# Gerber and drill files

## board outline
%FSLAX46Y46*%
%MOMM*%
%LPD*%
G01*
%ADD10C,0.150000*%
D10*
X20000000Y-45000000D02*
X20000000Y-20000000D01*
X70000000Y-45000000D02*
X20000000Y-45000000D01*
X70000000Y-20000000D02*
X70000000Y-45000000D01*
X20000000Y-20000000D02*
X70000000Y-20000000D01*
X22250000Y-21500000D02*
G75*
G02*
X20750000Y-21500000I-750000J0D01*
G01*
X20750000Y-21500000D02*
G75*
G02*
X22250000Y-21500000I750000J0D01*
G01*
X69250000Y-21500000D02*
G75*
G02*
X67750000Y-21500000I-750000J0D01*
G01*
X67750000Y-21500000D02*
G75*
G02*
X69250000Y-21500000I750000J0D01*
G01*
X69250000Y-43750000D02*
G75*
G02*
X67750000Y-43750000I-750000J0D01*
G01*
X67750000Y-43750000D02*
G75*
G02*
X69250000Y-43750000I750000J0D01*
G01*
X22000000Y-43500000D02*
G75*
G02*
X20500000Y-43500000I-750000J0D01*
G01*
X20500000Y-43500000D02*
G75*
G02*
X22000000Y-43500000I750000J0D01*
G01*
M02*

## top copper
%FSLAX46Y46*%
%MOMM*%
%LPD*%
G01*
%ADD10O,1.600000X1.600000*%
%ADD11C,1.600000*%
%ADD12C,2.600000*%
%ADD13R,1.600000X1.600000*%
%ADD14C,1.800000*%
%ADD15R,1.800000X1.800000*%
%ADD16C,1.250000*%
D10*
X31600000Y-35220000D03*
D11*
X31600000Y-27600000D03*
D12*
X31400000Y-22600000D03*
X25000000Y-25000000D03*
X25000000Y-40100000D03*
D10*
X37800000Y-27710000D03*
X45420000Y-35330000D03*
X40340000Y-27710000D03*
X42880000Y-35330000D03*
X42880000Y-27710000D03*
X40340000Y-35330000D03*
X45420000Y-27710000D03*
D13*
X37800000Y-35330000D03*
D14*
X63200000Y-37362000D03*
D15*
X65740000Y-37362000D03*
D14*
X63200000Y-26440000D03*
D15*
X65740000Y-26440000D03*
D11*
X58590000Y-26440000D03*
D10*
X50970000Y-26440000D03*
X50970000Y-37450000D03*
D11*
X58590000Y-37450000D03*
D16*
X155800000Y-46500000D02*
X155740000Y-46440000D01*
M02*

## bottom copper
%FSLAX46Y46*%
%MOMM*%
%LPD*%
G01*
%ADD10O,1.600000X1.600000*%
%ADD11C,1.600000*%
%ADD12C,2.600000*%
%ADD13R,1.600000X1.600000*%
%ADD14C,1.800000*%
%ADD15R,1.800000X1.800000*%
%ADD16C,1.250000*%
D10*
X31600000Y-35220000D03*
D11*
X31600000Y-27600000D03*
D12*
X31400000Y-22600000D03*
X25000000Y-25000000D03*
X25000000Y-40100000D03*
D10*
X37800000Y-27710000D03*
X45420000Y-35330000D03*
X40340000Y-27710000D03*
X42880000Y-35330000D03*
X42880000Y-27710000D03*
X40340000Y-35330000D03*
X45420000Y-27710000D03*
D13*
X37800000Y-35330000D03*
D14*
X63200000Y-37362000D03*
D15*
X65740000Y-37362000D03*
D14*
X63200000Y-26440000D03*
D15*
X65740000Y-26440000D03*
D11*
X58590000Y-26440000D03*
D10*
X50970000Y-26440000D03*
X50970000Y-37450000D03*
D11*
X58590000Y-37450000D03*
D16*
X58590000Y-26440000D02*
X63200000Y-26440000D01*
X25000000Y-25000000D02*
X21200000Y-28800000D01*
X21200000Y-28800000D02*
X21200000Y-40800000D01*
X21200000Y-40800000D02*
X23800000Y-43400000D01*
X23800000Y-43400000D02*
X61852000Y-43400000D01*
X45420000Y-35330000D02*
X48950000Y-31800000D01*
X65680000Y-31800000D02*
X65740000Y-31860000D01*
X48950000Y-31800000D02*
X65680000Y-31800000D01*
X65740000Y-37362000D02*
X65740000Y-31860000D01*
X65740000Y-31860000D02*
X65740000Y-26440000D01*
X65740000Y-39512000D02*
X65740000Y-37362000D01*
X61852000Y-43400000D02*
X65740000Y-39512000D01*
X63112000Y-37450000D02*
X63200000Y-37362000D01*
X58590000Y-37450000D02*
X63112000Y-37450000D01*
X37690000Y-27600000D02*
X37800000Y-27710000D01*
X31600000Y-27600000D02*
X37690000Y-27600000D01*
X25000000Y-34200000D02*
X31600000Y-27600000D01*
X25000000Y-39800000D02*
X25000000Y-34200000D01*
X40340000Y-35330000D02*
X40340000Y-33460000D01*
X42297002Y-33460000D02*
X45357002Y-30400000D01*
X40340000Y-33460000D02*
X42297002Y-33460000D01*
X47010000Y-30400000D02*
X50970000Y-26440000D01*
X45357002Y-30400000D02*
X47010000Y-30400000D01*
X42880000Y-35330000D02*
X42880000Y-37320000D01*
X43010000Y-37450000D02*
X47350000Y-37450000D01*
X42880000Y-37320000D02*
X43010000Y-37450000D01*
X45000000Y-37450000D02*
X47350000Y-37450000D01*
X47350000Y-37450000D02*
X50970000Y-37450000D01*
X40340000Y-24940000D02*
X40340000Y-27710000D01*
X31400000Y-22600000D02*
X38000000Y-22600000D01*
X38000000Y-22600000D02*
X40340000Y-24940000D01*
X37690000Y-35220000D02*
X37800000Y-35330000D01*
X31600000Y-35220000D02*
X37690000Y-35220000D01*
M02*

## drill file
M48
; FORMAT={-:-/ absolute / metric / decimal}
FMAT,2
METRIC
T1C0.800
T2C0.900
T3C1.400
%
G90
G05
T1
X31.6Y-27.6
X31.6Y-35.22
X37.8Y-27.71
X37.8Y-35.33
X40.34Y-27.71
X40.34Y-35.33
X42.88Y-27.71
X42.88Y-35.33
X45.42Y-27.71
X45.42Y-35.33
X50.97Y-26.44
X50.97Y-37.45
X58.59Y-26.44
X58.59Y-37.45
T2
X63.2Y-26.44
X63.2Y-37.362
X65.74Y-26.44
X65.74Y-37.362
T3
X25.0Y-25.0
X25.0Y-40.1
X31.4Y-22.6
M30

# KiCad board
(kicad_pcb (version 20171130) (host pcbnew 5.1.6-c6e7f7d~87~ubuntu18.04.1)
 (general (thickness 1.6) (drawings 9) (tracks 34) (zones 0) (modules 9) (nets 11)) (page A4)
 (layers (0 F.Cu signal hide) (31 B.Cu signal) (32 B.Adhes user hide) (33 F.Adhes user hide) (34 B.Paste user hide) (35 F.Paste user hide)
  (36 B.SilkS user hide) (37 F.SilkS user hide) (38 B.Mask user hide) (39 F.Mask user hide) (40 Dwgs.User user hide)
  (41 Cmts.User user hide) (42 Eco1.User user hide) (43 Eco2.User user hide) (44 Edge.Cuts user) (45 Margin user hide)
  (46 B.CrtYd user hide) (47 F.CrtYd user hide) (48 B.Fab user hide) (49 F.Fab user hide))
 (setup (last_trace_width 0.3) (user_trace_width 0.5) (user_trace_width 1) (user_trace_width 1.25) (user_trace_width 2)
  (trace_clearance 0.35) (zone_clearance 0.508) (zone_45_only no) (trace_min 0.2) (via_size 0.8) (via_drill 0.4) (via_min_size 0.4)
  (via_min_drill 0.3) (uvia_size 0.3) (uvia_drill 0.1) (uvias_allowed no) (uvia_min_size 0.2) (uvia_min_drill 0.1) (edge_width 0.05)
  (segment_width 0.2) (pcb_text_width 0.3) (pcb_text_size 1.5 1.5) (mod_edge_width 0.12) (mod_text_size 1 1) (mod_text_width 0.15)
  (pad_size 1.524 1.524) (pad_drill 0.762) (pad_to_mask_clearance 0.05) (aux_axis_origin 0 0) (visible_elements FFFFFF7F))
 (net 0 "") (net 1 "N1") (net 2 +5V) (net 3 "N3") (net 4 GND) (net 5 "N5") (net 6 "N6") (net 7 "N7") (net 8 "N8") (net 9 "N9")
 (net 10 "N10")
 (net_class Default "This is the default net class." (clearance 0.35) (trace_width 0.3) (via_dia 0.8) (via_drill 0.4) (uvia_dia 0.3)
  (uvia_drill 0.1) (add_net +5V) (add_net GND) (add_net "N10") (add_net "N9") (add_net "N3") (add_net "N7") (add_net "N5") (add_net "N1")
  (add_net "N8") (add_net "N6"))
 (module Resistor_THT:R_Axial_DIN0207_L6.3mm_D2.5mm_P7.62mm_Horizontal (layer F.Cu) (at 31.6 27.6 270)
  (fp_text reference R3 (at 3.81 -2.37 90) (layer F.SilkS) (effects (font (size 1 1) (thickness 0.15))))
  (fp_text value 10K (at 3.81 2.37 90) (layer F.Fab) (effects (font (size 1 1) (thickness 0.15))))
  (pad 2 thru_hole oval (at 7.62 0 270) (size 1.6 1.6) (drill 0.8) (layers *.Cu *.Mask) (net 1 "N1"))
  (pad 1 thru_hole circle (at 0 0 270) (size 1.6 1.6) (drill 0.8) (layers *.Cu *.Mask) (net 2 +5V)))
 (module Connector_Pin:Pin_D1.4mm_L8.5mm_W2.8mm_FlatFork (layer F.Cu) (at 31.4 22.6)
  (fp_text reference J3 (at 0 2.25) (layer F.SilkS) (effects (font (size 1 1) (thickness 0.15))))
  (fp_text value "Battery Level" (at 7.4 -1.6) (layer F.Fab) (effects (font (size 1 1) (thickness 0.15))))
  (pad 1 thru_hole circle (at 0 0) (size 2.6 2.6) (drill 1.4) (layers *.Cu *.Mask) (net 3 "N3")))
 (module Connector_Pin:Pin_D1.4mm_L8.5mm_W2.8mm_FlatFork (layer F.Cu) (at 25 25)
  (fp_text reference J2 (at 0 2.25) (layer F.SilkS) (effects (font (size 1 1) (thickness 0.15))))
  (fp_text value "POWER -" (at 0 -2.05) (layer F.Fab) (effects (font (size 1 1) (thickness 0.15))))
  (pad 1 thru_hole circle (at 0 0) (size 2.6 2.6) (drill 1.4) (layers *.Cu *.Mask) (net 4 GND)))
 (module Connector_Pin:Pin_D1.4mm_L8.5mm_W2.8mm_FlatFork (layer F.Cu) (at 25 40.1)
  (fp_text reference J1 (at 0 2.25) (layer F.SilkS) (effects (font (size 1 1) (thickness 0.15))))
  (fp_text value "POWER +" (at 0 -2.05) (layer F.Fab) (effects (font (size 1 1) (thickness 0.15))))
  (pad 1 thru_hole circle (at 0 0) (size 2.6 2.6) (drill 1.4) (layers *.Cu *.Mask) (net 2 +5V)))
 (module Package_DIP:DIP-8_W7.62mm (layer F.Cu) (at 37.8 35.33 90)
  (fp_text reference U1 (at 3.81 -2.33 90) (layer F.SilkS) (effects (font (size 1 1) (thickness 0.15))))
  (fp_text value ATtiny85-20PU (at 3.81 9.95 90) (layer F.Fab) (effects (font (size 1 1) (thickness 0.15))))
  (pad 8 thru_hole oval (at 7.62 0 90) (size 1.6 1.6) (drill 0.8) (layers *.Cu *.Mask) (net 2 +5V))
  (pad 4 thru_hole oval (at 0 7.62 90) (size 1.6 1.6) (drill 0.8) (layers *.Cu *.Mask) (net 4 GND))
  (pad 7 thru_hole oval (at 7.62 2.54 90) (size 1.6 1.6) (drill 0.8) (layers *.Cu *.Mask) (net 3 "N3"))
  (pad 3 thru_hole oval (at 0 5.08 90) (size 1.6 1.6) (drill 0.8) (layers *.Cu *.Mask) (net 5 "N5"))
  (pad 6 thru_hole oval (at 7.62 5.08 90) (size 1.6 1.6) (drill 0.8) (layers *.Cu *.Mask) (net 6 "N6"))
  (pad 2 thru_hole oval (at 0 2.54 90) (size 1.6 1.6) (drill 0.8) (layers *.Cu *.Mask) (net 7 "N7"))
  (pad 5 thru_hole oval (at 7.62 7.62 90) (size 1.6 1.6) (drill 0.8) (layers *.Cu *.Mask) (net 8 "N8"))
  (pad 1 thru_hole rect (at 0 0 90) (size 1.6 1.6) (drill 0.8) (layers *.Cu *.Mask) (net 1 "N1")))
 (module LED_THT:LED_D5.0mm (layer F.Cu) (at 65.74 37.362 180)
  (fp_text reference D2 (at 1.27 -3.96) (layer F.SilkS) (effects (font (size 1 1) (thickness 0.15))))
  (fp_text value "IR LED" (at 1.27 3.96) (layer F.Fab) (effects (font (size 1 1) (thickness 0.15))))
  (pad 2 thru_hole circle (at 2.54 0 180) (size 1.8 1.8) (drill 0.9) (layers *.Cu *.Mask) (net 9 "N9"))
  (pad 1 thru_hole rect (at 0 0 180) (size 1.8 1.8) (drill 0.9) (layers *.Cu *.Mask) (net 4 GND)))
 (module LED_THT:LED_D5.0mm (layer F.Cu) (at 65.74 26.44 180)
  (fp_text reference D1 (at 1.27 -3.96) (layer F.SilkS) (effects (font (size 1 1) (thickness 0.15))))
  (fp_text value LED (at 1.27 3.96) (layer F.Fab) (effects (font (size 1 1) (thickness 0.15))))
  (pad 2 thru_hole circle (at 2.54 0 180) (size 1.8 1.8) (drill 0.9) (layers *.Cu *.Mask) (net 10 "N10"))
  (pad 1 thru_hole rect (at 0 0 180) (size 1.8 1.8) (drill 0.9) (layers *.Cu *.Mask) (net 4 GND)))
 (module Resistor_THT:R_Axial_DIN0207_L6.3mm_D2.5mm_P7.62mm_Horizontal (layer F.Cu) (at 58.59 26.44 180)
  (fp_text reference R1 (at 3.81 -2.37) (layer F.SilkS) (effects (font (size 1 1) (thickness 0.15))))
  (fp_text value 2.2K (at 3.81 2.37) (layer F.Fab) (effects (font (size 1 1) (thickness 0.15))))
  (pad 1 thru_hole circle (at 0 0 180) (size 1.6 1.6) (drill 0.8) (layers *.Cu *.Mask) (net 10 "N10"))
  (pad 2 thru_hole oval (at 7.62 0 180) (size 1.6 1.6) (drill 0.8) (layers *.Cu *.Mask) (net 7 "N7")))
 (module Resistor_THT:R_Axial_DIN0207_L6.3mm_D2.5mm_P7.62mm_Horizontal (layer F.Cu) (at 58.59 37.45 180)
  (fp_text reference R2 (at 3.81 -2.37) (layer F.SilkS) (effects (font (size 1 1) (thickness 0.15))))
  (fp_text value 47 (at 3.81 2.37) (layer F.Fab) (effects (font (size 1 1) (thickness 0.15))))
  (pad 2 thru_hole oval (at 7.62 0 180) (size 1.6 1.6) (drill 0.8) (layers *.Cu *.Mask) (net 5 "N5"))
  (pad 1 thru_hole circle (at 0 0 180) (size 1.6 1.6) (drill 0.8) (layers *.Cu *.Mask) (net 9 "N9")))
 (gr_line (start 20 45) (end 20 20) (layer Edge.Cuts) (width 0.15))
 (gr_line (start 70 45) (end 20 45) (layer Edge.Cuts) (width 0.15))
 (gr_line (start 70 20) (end 70 45) (layer Edge.Cuts) (width 0.15))
 (gr_line (start 20 20) (end 70 20) (layer Edge.Cuts) (width 0.15))
 (gr_circle (center 21.5 21.5) (end 22.25 21.5) (layer Edge.Cuts) (width 0.15))
 (gr_circle (center 68.5 21.5) (end 69.25 21.5) (layer Edge.Cuts) (width 0.15))
 (gr_circle (center 68.5 43.75) (end 69.25 43.75) (layer Edge.Cuts) (width 0.15))
 (gr_circle (center 21.25 43.5) (end 22 43.5) (layer Edge.Cuts) (width 0.15))
 (segment (start 58.59 26.44) (end 63.2 26.44) (width 1.25) (layer B.Cu) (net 10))
 (segment (start 155.8 46.5) (end 155.74 46.44) (width 1.25) (layer F.Cu) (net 4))
 (segment (start 25 25) (end 21.2 28.8) (width 1.25) (layer B.Cu) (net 4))
 (segment (start 21.2 28.8) (end 21.2 40.8) (width 1.25) (layer B.Cu) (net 4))
 (segment (start 21.2 40.8) (end 23.8 43.4) (width 1.25) (layer B.Cu) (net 4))
 (segment (start 23.8 43.4) (end 61.852 43.4) (width 1.25) (layer B.Cu) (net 4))
 (segment (start 45.42 35.33) (end 48.95 31.8) (width 1.25) (layer B.Cu) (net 4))
 (segment (start 65.68 31.8) (end 65.74 31.86) (width 1.25) (layer B.Cu) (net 4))
 (segment (start 48.95 31.8) (end 65.68 31.8) (width 1.25) (layer B.Cu) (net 4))
 (segment (start 65.74 37.362) (end 65.74 31.86) (width 1.25) (layer B.Cu) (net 4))
 (segment (start 65.74 31.86) (end 65.74 26.44) (width 1.25) (layer B.Cu) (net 4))
 (segment (start 65.74 39.512) (end 65.74 37.362) (width 1.25) (layer B.Cu) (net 4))
 (segment (start 61.852 43.4) (end 65.74 39.512) (width 1.25) (layer B.Cu) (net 4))
 (segment (start 63.112 37.45) (end 63.2 37.362) (width 1.25) (layer B.Cu) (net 9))
 (segment (start 58.59 37.45) (end 63.112 37.45) (width 1.25) (layer B.Cu) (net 9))
 (segment (start 37.69 27.6) (end 37.8 27.71) (width 1.25) (layer B.Cu) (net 2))
 (segment (start 31.6 27.6) (end 37.69 27.6) (width 1.25) (layer B.Cu) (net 2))
 (segment (start 25 34.2) (end 31.6 27.6) (width 1.25) (layer B.Cu) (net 2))
 (segment (start 25 39.8) (end 25 34.2) (width 1.25) (layer B.Cu) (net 2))
 (segment (start 40.34 35.33) (end 40.34 33.46) (width 1.25) (layer B.Cu) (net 7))
 (segment (start 42.297002 33.46) (end 45.357002 30.4) (width 1.25) (layer B.Cu) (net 7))
 (segment (start 40.34 33.46) (end 42.297002 33.46) (width 1.25) (layer B.Cu) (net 7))
 (segment (start 47.01 30.4) (end 50.97 26.44) (width 1.25) (layer B.Cu) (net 7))
 (segment (start 45.357002 30.4) (end 47.01 30.4) (width 1.25) (layer B.Cu) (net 7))
 (segment (start 42.88 35.33) (end 42.88 37.32) (width 1.25) (layer B.Cu) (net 5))
 (segment (start 43.01 37.45) (end 47.35 37.45) (width 1.25) (layer B.Cu) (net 5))
 (segment (start 42.88 37.32) (end 43.01 37.45) (width 1.25) (layer B.Cu) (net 5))
 (segment (start 45 37.45) (end 47.35 37.45) (width 1.25) (layer B.Cu) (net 5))
 (segment (start 47.35 37.45) (end 50.97 37.45) (width 1.25) (layer B.Cu) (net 5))
 (segment (start 40.34 24.94) (end 40.34 27.71) (width 1.25) (layer B.Cu) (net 3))
 (segment (start 31.4 22.6) (end 38 22.6) (width 1.25) (layer B.Cu) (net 3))
 (segment (start 38 22.6) (end 40.34 24.94) (width 1.25) (layer B.Cu) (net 3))
 (segment (start 37.69 35.22) (end 37.8 35.33) (width 1.25) (layer B.Cu) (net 1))
 (segment (start 31.6 35.22) (end 37.69 35.22) (width 1.25) (layer B.Cu) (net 1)))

